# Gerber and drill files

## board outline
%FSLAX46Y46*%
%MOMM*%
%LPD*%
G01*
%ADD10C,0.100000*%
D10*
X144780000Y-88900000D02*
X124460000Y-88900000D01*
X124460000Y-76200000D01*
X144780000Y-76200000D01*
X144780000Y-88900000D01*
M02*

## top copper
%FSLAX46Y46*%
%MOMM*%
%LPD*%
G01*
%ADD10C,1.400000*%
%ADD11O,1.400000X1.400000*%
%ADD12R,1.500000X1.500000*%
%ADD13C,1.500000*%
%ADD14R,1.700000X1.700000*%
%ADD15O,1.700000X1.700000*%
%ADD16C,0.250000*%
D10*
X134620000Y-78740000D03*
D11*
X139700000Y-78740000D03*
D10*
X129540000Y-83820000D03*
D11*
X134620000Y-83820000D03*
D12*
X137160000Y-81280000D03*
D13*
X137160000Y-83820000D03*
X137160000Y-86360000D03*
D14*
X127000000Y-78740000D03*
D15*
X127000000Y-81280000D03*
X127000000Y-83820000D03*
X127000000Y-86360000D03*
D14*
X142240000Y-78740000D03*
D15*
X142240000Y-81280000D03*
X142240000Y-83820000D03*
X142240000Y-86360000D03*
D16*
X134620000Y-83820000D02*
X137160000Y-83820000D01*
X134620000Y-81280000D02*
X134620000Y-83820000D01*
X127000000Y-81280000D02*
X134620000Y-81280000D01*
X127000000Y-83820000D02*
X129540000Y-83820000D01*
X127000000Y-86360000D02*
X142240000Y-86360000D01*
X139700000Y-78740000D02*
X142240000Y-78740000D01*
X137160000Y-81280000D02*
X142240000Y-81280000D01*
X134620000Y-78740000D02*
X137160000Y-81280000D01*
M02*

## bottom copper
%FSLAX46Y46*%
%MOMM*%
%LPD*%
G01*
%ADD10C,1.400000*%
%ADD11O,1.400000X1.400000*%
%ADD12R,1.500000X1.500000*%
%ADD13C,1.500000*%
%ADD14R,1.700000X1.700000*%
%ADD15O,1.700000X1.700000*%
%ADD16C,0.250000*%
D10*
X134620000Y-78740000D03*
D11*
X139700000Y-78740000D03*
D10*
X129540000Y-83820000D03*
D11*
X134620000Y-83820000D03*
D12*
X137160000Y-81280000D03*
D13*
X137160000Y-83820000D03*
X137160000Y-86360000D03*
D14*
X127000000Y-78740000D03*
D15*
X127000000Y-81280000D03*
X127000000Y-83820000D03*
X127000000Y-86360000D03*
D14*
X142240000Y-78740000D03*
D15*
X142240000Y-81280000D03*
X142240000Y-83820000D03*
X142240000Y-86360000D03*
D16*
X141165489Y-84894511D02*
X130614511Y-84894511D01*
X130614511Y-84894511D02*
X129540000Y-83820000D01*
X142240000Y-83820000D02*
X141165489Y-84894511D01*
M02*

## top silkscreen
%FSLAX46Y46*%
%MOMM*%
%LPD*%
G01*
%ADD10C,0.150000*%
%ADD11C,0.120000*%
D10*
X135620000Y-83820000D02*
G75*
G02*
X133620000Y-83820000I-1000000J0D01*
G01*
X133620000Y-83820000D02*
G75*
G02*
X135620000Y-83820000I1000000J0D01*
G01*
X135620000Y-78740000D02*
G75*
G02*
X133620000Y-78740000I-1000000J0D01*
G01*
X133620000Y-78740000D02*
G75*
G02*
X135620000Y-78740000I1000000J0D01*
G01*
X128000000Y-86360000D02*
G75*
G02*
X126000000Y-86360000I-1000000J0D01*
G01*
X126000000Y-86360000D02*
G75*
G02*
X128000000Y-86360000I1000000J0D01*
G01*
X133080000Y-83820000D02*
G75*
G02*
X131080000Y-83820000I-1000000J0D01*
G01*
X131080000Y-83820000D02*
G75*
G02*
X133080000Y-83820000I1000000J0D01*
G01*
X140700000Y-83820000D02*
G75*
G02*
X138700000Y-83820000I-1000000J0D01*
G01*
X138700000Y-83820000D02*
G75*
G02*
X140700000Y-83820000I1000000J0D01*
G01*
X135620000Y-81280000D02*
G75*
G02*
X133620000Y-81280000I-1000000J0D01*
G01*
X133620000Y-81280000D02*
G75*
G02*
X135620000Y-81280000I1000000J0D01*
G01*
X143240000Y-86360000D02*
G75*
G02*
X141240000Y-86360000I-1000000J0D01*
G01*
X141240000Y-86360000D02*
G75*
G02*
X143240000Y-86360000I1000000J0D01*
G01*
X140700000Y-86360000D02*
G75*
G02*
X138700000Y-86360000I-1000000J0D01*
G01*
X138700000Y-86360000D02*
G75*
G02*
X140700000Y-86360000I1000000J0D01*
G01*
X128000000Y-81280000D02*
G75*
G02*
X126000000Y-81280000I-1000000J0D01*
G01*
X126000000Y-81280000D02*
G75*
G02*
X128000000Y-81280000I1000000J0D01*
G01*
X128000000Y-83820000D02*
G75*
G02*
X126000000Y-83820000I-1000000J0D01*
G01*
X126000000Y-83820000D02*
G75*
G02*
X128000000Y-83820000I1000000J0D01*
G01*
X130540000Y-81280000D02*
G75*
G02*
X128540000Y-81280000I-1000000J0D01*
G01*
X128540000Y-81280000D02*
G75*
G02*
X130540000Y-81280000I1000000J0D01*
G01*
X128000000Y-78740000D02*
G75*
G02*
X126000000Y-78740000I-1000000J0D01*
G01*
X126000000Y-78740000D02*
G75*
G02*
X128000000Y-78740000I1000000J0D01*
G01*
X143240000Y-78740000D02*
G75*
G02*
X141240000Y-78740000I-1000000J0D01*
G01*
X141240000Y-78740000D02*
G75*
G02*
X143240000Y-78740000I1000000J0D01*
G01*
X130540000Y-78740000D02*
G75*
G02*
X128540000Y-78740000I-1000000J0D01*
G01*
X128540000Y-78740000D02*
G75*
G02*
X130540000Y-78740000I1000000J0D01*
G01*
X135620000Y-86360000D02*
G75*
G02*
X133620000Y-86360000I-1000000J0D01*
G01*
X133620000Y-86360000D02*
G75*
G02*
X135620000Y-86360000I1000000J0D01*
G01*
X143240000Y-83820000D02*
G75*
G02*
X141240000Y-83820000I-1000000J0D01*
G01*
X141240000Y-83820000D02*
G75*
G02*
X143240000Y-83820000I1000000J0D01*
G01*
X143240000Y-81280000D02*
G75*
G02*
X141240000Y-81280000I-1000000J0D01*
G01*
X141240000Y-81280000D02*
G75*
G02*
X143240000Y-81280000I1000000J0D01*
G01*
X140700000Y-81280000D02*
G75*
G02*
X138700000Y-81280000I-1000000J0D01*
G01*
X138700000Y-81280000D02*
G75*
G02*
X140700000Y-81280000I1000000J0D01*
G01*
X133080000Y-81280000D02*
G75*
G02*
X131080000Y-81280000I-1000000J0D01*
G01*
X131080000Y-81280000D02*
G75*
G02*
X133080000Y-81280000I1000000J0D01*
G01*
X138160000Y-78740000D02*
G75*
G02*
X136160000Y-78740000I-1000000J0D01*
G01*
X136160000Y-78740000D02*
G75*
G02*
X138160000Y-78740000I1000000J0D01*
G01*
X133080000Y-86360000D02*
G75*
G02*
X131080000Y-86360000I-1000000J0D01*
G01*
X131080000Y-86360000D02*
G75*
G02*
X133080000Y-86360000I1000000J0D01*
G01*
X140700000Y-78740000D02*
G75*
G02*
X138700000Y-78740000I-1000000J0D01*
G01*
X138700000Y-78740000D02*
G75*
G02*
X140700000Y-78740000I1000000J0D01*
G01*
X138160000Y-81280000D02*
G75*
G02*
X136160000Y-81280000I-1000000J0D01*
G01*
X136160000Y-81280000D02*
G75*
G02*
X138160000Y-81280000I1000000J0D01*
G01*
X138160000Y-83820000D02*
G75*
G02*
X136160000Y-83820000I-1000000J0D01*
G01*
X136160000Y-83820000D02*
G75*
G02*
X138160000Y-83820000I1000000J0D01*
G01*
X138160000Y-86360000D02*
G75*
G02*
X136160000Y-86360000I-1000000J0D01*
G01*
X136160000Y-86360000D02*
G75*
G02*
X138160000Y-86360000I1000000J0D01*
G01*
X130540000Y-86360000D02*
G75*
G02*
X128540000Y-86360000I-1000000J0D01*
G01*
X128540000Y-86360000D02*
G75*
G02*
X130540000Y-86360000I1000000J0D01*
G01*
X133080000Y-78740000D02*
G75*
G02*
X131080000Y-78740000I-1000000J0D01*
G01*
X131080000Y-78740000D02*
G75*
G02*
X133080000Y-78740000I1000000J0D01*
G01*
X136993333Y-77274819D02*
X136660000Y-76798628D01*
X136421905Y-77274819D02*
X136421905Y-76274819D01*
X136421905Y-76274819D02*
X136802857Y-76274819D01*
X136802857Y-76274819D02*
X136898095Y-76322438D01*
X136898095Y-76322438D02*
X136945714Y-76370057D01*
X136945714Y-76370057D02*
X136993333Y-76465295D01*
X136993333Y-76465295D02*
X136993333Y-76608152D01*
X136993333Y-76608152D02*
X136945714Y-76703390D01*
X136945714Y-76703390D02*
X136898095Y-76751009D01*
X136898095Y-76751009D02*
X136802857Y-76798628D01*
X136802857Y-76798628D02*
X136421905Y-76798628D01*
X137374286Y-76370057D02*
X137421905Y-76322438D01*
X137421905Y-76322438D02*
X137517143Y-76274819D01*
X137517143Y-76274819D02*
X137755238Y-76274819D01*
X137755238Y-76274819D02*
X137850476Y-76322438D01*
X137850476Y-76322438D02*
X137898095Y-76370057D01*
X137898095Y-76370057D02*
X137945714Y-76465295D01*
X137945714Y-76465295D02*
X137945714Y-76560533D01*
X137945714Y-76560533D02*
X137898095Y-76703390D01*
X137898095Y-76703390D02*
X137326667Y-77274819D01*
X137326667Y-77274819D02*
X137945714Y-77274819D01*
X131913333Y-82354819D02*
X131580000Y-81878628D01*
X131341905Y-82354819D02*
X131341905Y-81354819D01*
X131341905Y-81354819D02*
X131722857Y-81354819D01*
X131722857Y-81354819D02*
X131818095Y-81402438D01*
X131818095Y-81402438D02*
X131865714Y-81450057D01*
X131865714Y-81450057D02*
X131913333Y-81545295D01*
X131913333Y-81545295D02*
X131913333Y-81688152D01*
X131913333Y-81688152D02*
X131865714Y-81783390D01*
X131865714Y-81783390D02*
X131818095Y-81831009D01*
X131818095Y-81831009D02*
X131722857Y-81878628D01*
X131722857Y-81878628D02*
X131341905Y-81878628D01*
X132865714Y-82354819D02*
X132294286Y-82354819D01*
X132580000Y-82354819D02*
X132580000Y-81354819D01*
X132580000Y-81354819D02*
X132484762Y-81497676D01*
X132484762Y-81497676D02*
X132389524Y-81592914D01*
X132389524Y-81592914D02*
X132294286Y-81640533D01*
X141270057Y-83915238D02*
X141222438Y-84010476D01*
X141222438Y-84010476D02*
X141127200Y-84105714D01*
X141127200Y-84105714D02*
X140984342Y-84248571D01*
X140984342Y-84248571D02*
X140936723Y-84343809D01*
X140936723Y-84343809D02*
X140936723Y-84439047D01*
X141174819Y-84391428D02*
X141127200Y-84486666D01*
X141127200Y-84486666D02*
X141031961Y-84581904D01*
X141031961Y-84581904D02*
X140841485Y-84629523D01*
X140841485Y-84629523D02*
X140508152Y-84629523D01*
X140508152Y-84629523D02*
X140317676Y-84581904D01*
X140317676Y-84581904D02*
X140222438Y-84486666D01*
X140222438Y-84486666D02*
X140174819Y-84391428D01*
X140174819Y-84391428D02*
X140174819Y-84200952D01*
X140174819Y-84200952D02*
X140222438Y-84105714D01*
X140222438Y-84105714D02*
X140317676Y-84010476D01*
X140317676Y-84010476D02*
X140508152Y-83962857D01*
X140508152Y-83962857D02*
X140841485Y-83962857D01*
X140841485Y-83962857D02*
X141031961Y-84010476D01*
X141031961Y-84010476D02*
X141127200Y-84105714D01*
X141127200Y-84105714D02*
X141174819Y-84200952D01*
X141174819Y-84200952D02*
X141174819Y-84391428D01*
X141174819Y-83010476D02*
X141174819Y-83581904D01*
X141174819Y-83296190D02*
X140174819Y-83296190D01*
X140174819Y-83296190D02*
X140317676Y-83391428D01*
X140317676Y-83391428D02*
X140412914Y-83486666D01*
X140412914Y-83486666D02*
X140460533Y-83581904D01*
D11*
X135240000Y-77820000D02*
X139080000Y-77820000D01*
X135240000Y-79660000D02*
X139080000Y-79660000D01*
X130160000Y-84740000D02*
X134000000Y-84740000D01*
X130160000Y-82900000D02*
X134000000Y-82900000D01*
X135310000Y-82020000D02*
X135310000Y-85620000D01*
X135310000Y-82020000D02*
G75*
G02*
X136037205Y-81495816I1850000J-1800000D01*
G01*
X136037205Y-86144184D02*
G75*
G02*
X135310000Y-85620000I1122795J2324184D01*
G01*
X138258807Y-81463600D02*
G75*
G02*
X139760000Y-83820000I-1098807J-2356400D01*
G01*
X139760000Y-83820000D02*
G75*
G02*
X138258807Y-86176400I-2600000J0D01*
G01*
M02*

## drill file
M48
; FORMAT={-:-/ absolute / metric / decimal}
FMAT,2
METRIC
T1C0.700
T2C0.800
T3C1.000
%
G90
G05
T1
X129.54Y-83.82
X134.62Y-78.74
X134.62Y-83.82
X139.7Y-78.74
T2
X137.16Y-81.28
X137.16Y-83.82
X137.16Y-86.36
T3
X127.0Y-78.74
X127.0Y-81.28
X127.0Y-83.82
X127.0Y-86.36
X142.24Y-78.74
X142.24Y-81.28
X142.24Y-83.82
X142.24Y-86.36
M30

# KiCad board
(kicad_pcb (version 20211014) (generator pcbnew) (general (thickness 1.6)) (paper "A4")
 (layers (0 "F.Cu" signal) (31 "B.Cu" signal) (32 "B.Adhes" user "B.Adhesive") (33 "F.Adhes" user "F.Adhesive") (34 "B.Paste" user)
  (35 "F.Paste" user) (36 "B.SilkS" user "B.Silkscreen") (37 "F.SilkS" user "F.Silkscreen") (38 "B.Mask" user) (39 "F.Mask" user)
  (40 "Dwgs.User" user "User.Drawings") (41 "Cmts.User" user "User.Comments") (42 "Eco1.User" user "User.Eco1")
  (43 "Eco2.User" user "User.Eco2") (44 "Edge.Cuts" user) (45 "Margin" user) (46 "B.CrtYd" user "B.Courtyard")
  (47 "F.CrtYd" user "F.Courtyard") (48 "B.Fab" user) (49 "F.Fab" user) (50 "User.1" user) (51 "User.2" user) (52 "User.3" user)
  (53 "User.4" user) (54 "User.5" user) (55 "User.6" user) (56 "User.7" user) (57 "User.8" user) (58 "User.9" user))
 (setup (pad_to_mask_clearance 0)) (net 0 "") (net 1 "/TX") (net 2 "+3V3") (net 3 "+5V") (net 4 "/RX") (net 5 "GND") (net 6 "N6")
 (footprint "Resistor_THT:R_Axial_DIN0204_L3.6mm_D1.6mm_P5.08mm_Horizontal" (layer "F.Cu") (at 134.62 78.74)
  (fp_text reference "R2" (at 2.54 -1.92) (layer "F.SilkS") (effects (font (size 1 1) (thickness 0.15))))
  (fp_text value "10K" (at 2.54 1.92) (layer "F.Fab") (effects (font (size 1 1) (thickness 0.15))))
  (fp_line (start 0.62 -0.92) (end 4.46 -0.92) (layer "F.SilkS") (width 0.12))
  (fp_line (start 0.62 0.92) (end 4.46 0.92) (layer "F.SilkS") (width 0.12))
  (pad "1" thru_hole circle (at 0 0) (size 1.4 1.4) (drill 0.7) (layers *.Cu *.Mask) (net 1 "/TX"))
  (pad "2" thru_hole oval (at 5.08 0) (size 1.4 1.4) (drill 0.7) (layers *.Cu *.Mask) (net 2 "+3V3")))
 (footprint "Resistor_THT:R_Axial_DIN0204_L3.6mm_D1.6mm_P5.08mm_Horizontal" (layer "F.Cu") (at 129.54 83.82)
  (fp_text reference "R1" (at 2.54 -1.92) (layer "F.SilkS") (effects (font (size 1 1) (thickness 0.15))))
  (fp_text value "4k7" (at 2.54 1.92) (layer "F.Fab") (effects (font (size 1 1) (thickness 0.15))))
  (fp_line (start 0.62 0.92) (end 4.46 0.92) (layer "F.SilkS") (width 0.12))
  (fp_line (start 0.62 -0.92) (end 4.46 -0.92) (layer "F.SilkS") (width 0.12))
  (pad "1" thru_hole circle (at 0 0) (size 1.4 1.4) (drill 0.7) (layers *.Cu *.Mask) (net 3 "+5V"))
  (pad "2" thru_hole oval (at 5.08 0) (size 1.4 1.4) (drill 0.7) (layers *.Cu *.Mask) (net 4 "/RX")))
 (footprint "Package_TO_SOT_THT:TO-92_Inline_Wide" (layer "F.Cu") (at 137.16 81.28 -90)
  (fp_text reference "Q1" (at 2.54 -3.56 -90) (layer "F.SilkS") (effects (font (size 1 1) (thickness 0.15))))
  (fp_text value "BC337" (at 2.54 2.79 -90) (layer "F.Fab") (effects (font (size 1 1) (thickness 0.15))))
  (fp_line (start 0.74 1.85) (end 4.34 1.85) (layer "F.SilkS") (width 0.12))
  (fp_arc (start 0.74 1.85) (mid 0.446097 1.509328) (end 0.215816 1.122795) (layer "F.SilkS") (width 0.12))
  (fp_arc (start 4.864184 1.122795) (mid 4.633903 1.509328) (end 4.34 1.85) (layer "F.SilkS") (width 0.12))
  (fp_arc (start 0.1836 -1.098807) (mid 1.143021 -2.192817) (end 2.54 -2.6) (layer "F.SilkS") (width 0.12))
  (fp_arc (start 2.54 -2.6) (mid 3.936979 -2.192818) (end 4.8964 -1.098807) (layer "F.SilkS") (width 0.12))
  (pad "1" thru_hole rect (at 0 0 270) (size 1.5 1.5) (drill 0.8) (layers *.Cu *.Mask) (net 1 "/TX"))
  (pad "2" thru_hole circle (at 2.54 0 270) (size 1.5 1.5) (drill 0.8) (layers *.Cu *.Mask) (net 4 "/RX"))
  (pad "3" thru_hole circle (at 5.08 0 270) (size 1.5 1.5) (drill 0.8) (layers *.Cu *.Mask) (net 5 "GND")))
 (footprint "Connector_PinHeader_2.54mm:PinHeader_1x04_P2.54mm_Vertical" (layer "B.Cu") (at 127 78.74 180)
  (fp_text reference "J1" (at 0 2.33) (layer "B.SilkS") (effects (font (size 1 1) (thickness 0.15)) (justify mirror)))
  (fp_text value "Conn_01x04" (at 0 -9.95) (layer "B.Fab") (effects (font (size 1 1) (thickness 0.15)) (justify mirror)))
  (pad "1" thru_hole rect (at 0 0 180) (size 1.7 1.7) (drill 1) (layers *.Cu *.Mask) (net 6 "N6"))
  (pad "2" thru_hole oval (at 0 -2.54 180) (size 1.7 1.7) (drill 1) (layers *.Cu *.Mask) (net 4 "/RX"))
  (pad "3" thru_hole oval (at 0 -5.08 180) (size 1.7 1.7) (drill 1) (layers *.Cu *.Mask) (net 3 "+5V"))
  (pad "4" thru_hole oval (at 0 -7.62 180) (size 1.7 1.7) (drill 1) (layers *.Cu *.Mask) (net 5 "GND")))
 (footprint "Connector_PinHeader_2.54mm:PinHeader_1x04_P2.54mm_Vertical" (layer "B.Cu") (at 142.24 78.74 180)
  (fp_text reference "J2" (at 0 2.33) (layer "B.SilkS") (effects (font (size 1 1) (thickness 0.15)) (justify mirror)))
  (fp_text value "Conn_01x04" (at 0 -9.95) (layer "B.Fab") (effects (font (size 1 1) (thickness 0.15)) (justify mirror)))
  (pad "1" thru_hole rect (at 0 0 180) (size 1.7 1.7) (drill 1) (layers *.Cu *.Mask) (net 2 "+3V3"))
  (pad "2" thru_hole oval (at 0 -2.54 180) (size 1.7 1.7) (drill 1) (layers *.Cu *.Mask) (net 1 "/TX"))
  (pad "3" thru_hole oval (at 0 -5.08 180) (size 1.7 1.7) (drill 1) (layers *.Cu *.Mask) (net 3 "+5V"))
  (pad "4" thru_hole oval (at 0 -7.62 180) (size 1.7 1.7) (drill 1) (layers *.Cu *.Mask) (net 5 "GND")))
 (gr_circle (center 134.62 83.82) (end 135.62 83.82) (layer "F.SilkS") (width 0.15) (fill none))
 (gr_circle (center 134.62 78.74) (end 135.62 78.74) (layer "F.SilkS") (width 0.15) (fill none))
 (gr_circle (center 127 86.36) (end 128 86.36) (layer "F.SilkS") (width 0.15) (fill none))
 (gr_circle (center 132.08 83.82) (end 133.08 83.82) (layer "F.SilkS") (width 0.15) (fill none))
 (gr_circle (center 139.7 83.82) (end 140.7 83.82) (layer "F.SilkS") (width 0.15) (fill none))
 (gr_circle (center 134.62 81.28) (end 135.62 81.28) (layer "F.SilkS") (width 0.15) (fill none))
 (gr_circle (center 142.24 86.36) (end 143.24 86.36) (layer "F.SilkS") (width 0.15) (fill none))
 (gr_circle (center 139.7 86.36) (end 140.7 86.36) (layer "F.SilkS") (width 0.15) (fill none))
 (gr_circle (center 127 81.28) (end 128 81.28) (layer "F.SilkS") (width 0.15) (fill none))
 (gr_circle (center 127 83.82) (end 128 83.82) (layer "F.SilkS") (width 0.15) (fill none))
 (gr_circle (center 129.54 81.28) (end 130.54 81.28) (layer "F.SilkS") (width 0.15) (fill none))
 (gr_circle (center 127 78.74) (end 128 78.74) (layer "F.SilkS") (width 0.15) (fill none))
 (gr_circle (center 142.24 78.74) (end 143.24 78.74) (layer "F.SilkS") (width 0.15) (fill none))
 (gr_circle (center 129.54 78.74) (end 130.54 78.74) (layer "F.SilkS") (width 0.15) (fill none))
 (gr_circle (center 134.62 86.36) (end 135.62 86.36) (layer "F.SilkS") (width 0.15) (fill none))
 (gr_circle (center 142.24 83.82) (end 143.24 83.82) (layer "F.SilkS") (width 0.15) (fill none))
 (gr_circle (center 142.24 81.28) (end 143.24 81.28) (layer "F.SilkS") (width 0.15) (fill none))
 (gr_circle (center 139.7 81.28) (end 140.7 81.28) (layer "F.SilkS") (width 0.15) (fill none))
 (gr_circle (center 132.08 81.28) (end 133.08 81.28) (layer "F.SilkS") (width 0.15) (fill none))
 (gr_circle (center 137.16 78.74) (end 138.16 78.74) (layer "F.SilkS") (width 0.15) (fill none))
 (gr_circle (center 132.08 86.36) (end 133.08 86.36) (layer "F.SilkS") (width 0.15) (fill none))
 (gr_circle (center 139.7 78.74) (end 140.7 78.74) (layer "F.SilkS") (width 0.15) (fill none))
 (gr_circle (center 137.16 81.28) (end 138.16 81.28) (layer "F.SilkS") (width 0.15) (fill none))
 (gr_circle (center 137.16 83.82) (end 138.16 83.82) (layer "F.SilkS") (width 0.15) (fill none))
 (gr_circle (center 137.16 86.36) (end 138.16 86.36) (layer "F.SilkS") (width 0.15) (fill none))
 (gr_circle (center 129.54 86.36) (end 130.54 86.36) (layer "F.SilkS") (width 0.15) (fill none))
 (gr_circle (center 132.08 78.74) (end 133.08 78.74) (layer "F.SilkS") (width 0.15) (fill none))
 (gr_poly (pts (xy 144.78 88.9) (xy 124.46 88.9) (xy 124.46 76.2) (xy 144.78 76.2)) (layer "Edge.Cuts") (width 0.1) (fill none))
 (segment (start 134.62 83.82) (end 137.16 83.82) (width 0.25) (layer "F.Cu") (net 4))
 (segment (start 134.62 81.28) (end 134.62 83.82) (width 0.25) (layer "F.Cu") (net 4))
 (segment (start 127 81.28) (end 134.62 81.28) (width 0.25) (layer "F.Cu") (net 4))
 (segment (start 127 83.82) (end 129.54 83.82) (width 0.25) (layer "F.Cu") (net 3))
 (segment (start 141.165489 84.894511) (end 130.614511 84.894511) (width 0.25) (layer "B.Cu") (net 3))
 (segment (start 130.614511 84.894511) (end 129.54 83.82) (width 0.25) (layer "B.Cu") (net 3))
 (segment (start 142.24 83.82) (end 141.165489 84.894511) (width 0.25) (layer "B.Cu") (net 3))
 (segment (start 127 86.36) (end 142.24 86.36) (width 0.25) (layer "F.Cu") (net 5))
 (segment (start 139.7 78.74) (end 142.24 78.74) (width 0.25) (layer "F.Cu") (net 2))
 (segment (start 137.16 81.28) (end 142.24 81.28) (width 0.25) (layer "F.Cu") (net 1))
 (segment (start 134.62 78.74) (end 137.16 81.28) (width 0.25) (layer "F.Cu") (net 1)))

